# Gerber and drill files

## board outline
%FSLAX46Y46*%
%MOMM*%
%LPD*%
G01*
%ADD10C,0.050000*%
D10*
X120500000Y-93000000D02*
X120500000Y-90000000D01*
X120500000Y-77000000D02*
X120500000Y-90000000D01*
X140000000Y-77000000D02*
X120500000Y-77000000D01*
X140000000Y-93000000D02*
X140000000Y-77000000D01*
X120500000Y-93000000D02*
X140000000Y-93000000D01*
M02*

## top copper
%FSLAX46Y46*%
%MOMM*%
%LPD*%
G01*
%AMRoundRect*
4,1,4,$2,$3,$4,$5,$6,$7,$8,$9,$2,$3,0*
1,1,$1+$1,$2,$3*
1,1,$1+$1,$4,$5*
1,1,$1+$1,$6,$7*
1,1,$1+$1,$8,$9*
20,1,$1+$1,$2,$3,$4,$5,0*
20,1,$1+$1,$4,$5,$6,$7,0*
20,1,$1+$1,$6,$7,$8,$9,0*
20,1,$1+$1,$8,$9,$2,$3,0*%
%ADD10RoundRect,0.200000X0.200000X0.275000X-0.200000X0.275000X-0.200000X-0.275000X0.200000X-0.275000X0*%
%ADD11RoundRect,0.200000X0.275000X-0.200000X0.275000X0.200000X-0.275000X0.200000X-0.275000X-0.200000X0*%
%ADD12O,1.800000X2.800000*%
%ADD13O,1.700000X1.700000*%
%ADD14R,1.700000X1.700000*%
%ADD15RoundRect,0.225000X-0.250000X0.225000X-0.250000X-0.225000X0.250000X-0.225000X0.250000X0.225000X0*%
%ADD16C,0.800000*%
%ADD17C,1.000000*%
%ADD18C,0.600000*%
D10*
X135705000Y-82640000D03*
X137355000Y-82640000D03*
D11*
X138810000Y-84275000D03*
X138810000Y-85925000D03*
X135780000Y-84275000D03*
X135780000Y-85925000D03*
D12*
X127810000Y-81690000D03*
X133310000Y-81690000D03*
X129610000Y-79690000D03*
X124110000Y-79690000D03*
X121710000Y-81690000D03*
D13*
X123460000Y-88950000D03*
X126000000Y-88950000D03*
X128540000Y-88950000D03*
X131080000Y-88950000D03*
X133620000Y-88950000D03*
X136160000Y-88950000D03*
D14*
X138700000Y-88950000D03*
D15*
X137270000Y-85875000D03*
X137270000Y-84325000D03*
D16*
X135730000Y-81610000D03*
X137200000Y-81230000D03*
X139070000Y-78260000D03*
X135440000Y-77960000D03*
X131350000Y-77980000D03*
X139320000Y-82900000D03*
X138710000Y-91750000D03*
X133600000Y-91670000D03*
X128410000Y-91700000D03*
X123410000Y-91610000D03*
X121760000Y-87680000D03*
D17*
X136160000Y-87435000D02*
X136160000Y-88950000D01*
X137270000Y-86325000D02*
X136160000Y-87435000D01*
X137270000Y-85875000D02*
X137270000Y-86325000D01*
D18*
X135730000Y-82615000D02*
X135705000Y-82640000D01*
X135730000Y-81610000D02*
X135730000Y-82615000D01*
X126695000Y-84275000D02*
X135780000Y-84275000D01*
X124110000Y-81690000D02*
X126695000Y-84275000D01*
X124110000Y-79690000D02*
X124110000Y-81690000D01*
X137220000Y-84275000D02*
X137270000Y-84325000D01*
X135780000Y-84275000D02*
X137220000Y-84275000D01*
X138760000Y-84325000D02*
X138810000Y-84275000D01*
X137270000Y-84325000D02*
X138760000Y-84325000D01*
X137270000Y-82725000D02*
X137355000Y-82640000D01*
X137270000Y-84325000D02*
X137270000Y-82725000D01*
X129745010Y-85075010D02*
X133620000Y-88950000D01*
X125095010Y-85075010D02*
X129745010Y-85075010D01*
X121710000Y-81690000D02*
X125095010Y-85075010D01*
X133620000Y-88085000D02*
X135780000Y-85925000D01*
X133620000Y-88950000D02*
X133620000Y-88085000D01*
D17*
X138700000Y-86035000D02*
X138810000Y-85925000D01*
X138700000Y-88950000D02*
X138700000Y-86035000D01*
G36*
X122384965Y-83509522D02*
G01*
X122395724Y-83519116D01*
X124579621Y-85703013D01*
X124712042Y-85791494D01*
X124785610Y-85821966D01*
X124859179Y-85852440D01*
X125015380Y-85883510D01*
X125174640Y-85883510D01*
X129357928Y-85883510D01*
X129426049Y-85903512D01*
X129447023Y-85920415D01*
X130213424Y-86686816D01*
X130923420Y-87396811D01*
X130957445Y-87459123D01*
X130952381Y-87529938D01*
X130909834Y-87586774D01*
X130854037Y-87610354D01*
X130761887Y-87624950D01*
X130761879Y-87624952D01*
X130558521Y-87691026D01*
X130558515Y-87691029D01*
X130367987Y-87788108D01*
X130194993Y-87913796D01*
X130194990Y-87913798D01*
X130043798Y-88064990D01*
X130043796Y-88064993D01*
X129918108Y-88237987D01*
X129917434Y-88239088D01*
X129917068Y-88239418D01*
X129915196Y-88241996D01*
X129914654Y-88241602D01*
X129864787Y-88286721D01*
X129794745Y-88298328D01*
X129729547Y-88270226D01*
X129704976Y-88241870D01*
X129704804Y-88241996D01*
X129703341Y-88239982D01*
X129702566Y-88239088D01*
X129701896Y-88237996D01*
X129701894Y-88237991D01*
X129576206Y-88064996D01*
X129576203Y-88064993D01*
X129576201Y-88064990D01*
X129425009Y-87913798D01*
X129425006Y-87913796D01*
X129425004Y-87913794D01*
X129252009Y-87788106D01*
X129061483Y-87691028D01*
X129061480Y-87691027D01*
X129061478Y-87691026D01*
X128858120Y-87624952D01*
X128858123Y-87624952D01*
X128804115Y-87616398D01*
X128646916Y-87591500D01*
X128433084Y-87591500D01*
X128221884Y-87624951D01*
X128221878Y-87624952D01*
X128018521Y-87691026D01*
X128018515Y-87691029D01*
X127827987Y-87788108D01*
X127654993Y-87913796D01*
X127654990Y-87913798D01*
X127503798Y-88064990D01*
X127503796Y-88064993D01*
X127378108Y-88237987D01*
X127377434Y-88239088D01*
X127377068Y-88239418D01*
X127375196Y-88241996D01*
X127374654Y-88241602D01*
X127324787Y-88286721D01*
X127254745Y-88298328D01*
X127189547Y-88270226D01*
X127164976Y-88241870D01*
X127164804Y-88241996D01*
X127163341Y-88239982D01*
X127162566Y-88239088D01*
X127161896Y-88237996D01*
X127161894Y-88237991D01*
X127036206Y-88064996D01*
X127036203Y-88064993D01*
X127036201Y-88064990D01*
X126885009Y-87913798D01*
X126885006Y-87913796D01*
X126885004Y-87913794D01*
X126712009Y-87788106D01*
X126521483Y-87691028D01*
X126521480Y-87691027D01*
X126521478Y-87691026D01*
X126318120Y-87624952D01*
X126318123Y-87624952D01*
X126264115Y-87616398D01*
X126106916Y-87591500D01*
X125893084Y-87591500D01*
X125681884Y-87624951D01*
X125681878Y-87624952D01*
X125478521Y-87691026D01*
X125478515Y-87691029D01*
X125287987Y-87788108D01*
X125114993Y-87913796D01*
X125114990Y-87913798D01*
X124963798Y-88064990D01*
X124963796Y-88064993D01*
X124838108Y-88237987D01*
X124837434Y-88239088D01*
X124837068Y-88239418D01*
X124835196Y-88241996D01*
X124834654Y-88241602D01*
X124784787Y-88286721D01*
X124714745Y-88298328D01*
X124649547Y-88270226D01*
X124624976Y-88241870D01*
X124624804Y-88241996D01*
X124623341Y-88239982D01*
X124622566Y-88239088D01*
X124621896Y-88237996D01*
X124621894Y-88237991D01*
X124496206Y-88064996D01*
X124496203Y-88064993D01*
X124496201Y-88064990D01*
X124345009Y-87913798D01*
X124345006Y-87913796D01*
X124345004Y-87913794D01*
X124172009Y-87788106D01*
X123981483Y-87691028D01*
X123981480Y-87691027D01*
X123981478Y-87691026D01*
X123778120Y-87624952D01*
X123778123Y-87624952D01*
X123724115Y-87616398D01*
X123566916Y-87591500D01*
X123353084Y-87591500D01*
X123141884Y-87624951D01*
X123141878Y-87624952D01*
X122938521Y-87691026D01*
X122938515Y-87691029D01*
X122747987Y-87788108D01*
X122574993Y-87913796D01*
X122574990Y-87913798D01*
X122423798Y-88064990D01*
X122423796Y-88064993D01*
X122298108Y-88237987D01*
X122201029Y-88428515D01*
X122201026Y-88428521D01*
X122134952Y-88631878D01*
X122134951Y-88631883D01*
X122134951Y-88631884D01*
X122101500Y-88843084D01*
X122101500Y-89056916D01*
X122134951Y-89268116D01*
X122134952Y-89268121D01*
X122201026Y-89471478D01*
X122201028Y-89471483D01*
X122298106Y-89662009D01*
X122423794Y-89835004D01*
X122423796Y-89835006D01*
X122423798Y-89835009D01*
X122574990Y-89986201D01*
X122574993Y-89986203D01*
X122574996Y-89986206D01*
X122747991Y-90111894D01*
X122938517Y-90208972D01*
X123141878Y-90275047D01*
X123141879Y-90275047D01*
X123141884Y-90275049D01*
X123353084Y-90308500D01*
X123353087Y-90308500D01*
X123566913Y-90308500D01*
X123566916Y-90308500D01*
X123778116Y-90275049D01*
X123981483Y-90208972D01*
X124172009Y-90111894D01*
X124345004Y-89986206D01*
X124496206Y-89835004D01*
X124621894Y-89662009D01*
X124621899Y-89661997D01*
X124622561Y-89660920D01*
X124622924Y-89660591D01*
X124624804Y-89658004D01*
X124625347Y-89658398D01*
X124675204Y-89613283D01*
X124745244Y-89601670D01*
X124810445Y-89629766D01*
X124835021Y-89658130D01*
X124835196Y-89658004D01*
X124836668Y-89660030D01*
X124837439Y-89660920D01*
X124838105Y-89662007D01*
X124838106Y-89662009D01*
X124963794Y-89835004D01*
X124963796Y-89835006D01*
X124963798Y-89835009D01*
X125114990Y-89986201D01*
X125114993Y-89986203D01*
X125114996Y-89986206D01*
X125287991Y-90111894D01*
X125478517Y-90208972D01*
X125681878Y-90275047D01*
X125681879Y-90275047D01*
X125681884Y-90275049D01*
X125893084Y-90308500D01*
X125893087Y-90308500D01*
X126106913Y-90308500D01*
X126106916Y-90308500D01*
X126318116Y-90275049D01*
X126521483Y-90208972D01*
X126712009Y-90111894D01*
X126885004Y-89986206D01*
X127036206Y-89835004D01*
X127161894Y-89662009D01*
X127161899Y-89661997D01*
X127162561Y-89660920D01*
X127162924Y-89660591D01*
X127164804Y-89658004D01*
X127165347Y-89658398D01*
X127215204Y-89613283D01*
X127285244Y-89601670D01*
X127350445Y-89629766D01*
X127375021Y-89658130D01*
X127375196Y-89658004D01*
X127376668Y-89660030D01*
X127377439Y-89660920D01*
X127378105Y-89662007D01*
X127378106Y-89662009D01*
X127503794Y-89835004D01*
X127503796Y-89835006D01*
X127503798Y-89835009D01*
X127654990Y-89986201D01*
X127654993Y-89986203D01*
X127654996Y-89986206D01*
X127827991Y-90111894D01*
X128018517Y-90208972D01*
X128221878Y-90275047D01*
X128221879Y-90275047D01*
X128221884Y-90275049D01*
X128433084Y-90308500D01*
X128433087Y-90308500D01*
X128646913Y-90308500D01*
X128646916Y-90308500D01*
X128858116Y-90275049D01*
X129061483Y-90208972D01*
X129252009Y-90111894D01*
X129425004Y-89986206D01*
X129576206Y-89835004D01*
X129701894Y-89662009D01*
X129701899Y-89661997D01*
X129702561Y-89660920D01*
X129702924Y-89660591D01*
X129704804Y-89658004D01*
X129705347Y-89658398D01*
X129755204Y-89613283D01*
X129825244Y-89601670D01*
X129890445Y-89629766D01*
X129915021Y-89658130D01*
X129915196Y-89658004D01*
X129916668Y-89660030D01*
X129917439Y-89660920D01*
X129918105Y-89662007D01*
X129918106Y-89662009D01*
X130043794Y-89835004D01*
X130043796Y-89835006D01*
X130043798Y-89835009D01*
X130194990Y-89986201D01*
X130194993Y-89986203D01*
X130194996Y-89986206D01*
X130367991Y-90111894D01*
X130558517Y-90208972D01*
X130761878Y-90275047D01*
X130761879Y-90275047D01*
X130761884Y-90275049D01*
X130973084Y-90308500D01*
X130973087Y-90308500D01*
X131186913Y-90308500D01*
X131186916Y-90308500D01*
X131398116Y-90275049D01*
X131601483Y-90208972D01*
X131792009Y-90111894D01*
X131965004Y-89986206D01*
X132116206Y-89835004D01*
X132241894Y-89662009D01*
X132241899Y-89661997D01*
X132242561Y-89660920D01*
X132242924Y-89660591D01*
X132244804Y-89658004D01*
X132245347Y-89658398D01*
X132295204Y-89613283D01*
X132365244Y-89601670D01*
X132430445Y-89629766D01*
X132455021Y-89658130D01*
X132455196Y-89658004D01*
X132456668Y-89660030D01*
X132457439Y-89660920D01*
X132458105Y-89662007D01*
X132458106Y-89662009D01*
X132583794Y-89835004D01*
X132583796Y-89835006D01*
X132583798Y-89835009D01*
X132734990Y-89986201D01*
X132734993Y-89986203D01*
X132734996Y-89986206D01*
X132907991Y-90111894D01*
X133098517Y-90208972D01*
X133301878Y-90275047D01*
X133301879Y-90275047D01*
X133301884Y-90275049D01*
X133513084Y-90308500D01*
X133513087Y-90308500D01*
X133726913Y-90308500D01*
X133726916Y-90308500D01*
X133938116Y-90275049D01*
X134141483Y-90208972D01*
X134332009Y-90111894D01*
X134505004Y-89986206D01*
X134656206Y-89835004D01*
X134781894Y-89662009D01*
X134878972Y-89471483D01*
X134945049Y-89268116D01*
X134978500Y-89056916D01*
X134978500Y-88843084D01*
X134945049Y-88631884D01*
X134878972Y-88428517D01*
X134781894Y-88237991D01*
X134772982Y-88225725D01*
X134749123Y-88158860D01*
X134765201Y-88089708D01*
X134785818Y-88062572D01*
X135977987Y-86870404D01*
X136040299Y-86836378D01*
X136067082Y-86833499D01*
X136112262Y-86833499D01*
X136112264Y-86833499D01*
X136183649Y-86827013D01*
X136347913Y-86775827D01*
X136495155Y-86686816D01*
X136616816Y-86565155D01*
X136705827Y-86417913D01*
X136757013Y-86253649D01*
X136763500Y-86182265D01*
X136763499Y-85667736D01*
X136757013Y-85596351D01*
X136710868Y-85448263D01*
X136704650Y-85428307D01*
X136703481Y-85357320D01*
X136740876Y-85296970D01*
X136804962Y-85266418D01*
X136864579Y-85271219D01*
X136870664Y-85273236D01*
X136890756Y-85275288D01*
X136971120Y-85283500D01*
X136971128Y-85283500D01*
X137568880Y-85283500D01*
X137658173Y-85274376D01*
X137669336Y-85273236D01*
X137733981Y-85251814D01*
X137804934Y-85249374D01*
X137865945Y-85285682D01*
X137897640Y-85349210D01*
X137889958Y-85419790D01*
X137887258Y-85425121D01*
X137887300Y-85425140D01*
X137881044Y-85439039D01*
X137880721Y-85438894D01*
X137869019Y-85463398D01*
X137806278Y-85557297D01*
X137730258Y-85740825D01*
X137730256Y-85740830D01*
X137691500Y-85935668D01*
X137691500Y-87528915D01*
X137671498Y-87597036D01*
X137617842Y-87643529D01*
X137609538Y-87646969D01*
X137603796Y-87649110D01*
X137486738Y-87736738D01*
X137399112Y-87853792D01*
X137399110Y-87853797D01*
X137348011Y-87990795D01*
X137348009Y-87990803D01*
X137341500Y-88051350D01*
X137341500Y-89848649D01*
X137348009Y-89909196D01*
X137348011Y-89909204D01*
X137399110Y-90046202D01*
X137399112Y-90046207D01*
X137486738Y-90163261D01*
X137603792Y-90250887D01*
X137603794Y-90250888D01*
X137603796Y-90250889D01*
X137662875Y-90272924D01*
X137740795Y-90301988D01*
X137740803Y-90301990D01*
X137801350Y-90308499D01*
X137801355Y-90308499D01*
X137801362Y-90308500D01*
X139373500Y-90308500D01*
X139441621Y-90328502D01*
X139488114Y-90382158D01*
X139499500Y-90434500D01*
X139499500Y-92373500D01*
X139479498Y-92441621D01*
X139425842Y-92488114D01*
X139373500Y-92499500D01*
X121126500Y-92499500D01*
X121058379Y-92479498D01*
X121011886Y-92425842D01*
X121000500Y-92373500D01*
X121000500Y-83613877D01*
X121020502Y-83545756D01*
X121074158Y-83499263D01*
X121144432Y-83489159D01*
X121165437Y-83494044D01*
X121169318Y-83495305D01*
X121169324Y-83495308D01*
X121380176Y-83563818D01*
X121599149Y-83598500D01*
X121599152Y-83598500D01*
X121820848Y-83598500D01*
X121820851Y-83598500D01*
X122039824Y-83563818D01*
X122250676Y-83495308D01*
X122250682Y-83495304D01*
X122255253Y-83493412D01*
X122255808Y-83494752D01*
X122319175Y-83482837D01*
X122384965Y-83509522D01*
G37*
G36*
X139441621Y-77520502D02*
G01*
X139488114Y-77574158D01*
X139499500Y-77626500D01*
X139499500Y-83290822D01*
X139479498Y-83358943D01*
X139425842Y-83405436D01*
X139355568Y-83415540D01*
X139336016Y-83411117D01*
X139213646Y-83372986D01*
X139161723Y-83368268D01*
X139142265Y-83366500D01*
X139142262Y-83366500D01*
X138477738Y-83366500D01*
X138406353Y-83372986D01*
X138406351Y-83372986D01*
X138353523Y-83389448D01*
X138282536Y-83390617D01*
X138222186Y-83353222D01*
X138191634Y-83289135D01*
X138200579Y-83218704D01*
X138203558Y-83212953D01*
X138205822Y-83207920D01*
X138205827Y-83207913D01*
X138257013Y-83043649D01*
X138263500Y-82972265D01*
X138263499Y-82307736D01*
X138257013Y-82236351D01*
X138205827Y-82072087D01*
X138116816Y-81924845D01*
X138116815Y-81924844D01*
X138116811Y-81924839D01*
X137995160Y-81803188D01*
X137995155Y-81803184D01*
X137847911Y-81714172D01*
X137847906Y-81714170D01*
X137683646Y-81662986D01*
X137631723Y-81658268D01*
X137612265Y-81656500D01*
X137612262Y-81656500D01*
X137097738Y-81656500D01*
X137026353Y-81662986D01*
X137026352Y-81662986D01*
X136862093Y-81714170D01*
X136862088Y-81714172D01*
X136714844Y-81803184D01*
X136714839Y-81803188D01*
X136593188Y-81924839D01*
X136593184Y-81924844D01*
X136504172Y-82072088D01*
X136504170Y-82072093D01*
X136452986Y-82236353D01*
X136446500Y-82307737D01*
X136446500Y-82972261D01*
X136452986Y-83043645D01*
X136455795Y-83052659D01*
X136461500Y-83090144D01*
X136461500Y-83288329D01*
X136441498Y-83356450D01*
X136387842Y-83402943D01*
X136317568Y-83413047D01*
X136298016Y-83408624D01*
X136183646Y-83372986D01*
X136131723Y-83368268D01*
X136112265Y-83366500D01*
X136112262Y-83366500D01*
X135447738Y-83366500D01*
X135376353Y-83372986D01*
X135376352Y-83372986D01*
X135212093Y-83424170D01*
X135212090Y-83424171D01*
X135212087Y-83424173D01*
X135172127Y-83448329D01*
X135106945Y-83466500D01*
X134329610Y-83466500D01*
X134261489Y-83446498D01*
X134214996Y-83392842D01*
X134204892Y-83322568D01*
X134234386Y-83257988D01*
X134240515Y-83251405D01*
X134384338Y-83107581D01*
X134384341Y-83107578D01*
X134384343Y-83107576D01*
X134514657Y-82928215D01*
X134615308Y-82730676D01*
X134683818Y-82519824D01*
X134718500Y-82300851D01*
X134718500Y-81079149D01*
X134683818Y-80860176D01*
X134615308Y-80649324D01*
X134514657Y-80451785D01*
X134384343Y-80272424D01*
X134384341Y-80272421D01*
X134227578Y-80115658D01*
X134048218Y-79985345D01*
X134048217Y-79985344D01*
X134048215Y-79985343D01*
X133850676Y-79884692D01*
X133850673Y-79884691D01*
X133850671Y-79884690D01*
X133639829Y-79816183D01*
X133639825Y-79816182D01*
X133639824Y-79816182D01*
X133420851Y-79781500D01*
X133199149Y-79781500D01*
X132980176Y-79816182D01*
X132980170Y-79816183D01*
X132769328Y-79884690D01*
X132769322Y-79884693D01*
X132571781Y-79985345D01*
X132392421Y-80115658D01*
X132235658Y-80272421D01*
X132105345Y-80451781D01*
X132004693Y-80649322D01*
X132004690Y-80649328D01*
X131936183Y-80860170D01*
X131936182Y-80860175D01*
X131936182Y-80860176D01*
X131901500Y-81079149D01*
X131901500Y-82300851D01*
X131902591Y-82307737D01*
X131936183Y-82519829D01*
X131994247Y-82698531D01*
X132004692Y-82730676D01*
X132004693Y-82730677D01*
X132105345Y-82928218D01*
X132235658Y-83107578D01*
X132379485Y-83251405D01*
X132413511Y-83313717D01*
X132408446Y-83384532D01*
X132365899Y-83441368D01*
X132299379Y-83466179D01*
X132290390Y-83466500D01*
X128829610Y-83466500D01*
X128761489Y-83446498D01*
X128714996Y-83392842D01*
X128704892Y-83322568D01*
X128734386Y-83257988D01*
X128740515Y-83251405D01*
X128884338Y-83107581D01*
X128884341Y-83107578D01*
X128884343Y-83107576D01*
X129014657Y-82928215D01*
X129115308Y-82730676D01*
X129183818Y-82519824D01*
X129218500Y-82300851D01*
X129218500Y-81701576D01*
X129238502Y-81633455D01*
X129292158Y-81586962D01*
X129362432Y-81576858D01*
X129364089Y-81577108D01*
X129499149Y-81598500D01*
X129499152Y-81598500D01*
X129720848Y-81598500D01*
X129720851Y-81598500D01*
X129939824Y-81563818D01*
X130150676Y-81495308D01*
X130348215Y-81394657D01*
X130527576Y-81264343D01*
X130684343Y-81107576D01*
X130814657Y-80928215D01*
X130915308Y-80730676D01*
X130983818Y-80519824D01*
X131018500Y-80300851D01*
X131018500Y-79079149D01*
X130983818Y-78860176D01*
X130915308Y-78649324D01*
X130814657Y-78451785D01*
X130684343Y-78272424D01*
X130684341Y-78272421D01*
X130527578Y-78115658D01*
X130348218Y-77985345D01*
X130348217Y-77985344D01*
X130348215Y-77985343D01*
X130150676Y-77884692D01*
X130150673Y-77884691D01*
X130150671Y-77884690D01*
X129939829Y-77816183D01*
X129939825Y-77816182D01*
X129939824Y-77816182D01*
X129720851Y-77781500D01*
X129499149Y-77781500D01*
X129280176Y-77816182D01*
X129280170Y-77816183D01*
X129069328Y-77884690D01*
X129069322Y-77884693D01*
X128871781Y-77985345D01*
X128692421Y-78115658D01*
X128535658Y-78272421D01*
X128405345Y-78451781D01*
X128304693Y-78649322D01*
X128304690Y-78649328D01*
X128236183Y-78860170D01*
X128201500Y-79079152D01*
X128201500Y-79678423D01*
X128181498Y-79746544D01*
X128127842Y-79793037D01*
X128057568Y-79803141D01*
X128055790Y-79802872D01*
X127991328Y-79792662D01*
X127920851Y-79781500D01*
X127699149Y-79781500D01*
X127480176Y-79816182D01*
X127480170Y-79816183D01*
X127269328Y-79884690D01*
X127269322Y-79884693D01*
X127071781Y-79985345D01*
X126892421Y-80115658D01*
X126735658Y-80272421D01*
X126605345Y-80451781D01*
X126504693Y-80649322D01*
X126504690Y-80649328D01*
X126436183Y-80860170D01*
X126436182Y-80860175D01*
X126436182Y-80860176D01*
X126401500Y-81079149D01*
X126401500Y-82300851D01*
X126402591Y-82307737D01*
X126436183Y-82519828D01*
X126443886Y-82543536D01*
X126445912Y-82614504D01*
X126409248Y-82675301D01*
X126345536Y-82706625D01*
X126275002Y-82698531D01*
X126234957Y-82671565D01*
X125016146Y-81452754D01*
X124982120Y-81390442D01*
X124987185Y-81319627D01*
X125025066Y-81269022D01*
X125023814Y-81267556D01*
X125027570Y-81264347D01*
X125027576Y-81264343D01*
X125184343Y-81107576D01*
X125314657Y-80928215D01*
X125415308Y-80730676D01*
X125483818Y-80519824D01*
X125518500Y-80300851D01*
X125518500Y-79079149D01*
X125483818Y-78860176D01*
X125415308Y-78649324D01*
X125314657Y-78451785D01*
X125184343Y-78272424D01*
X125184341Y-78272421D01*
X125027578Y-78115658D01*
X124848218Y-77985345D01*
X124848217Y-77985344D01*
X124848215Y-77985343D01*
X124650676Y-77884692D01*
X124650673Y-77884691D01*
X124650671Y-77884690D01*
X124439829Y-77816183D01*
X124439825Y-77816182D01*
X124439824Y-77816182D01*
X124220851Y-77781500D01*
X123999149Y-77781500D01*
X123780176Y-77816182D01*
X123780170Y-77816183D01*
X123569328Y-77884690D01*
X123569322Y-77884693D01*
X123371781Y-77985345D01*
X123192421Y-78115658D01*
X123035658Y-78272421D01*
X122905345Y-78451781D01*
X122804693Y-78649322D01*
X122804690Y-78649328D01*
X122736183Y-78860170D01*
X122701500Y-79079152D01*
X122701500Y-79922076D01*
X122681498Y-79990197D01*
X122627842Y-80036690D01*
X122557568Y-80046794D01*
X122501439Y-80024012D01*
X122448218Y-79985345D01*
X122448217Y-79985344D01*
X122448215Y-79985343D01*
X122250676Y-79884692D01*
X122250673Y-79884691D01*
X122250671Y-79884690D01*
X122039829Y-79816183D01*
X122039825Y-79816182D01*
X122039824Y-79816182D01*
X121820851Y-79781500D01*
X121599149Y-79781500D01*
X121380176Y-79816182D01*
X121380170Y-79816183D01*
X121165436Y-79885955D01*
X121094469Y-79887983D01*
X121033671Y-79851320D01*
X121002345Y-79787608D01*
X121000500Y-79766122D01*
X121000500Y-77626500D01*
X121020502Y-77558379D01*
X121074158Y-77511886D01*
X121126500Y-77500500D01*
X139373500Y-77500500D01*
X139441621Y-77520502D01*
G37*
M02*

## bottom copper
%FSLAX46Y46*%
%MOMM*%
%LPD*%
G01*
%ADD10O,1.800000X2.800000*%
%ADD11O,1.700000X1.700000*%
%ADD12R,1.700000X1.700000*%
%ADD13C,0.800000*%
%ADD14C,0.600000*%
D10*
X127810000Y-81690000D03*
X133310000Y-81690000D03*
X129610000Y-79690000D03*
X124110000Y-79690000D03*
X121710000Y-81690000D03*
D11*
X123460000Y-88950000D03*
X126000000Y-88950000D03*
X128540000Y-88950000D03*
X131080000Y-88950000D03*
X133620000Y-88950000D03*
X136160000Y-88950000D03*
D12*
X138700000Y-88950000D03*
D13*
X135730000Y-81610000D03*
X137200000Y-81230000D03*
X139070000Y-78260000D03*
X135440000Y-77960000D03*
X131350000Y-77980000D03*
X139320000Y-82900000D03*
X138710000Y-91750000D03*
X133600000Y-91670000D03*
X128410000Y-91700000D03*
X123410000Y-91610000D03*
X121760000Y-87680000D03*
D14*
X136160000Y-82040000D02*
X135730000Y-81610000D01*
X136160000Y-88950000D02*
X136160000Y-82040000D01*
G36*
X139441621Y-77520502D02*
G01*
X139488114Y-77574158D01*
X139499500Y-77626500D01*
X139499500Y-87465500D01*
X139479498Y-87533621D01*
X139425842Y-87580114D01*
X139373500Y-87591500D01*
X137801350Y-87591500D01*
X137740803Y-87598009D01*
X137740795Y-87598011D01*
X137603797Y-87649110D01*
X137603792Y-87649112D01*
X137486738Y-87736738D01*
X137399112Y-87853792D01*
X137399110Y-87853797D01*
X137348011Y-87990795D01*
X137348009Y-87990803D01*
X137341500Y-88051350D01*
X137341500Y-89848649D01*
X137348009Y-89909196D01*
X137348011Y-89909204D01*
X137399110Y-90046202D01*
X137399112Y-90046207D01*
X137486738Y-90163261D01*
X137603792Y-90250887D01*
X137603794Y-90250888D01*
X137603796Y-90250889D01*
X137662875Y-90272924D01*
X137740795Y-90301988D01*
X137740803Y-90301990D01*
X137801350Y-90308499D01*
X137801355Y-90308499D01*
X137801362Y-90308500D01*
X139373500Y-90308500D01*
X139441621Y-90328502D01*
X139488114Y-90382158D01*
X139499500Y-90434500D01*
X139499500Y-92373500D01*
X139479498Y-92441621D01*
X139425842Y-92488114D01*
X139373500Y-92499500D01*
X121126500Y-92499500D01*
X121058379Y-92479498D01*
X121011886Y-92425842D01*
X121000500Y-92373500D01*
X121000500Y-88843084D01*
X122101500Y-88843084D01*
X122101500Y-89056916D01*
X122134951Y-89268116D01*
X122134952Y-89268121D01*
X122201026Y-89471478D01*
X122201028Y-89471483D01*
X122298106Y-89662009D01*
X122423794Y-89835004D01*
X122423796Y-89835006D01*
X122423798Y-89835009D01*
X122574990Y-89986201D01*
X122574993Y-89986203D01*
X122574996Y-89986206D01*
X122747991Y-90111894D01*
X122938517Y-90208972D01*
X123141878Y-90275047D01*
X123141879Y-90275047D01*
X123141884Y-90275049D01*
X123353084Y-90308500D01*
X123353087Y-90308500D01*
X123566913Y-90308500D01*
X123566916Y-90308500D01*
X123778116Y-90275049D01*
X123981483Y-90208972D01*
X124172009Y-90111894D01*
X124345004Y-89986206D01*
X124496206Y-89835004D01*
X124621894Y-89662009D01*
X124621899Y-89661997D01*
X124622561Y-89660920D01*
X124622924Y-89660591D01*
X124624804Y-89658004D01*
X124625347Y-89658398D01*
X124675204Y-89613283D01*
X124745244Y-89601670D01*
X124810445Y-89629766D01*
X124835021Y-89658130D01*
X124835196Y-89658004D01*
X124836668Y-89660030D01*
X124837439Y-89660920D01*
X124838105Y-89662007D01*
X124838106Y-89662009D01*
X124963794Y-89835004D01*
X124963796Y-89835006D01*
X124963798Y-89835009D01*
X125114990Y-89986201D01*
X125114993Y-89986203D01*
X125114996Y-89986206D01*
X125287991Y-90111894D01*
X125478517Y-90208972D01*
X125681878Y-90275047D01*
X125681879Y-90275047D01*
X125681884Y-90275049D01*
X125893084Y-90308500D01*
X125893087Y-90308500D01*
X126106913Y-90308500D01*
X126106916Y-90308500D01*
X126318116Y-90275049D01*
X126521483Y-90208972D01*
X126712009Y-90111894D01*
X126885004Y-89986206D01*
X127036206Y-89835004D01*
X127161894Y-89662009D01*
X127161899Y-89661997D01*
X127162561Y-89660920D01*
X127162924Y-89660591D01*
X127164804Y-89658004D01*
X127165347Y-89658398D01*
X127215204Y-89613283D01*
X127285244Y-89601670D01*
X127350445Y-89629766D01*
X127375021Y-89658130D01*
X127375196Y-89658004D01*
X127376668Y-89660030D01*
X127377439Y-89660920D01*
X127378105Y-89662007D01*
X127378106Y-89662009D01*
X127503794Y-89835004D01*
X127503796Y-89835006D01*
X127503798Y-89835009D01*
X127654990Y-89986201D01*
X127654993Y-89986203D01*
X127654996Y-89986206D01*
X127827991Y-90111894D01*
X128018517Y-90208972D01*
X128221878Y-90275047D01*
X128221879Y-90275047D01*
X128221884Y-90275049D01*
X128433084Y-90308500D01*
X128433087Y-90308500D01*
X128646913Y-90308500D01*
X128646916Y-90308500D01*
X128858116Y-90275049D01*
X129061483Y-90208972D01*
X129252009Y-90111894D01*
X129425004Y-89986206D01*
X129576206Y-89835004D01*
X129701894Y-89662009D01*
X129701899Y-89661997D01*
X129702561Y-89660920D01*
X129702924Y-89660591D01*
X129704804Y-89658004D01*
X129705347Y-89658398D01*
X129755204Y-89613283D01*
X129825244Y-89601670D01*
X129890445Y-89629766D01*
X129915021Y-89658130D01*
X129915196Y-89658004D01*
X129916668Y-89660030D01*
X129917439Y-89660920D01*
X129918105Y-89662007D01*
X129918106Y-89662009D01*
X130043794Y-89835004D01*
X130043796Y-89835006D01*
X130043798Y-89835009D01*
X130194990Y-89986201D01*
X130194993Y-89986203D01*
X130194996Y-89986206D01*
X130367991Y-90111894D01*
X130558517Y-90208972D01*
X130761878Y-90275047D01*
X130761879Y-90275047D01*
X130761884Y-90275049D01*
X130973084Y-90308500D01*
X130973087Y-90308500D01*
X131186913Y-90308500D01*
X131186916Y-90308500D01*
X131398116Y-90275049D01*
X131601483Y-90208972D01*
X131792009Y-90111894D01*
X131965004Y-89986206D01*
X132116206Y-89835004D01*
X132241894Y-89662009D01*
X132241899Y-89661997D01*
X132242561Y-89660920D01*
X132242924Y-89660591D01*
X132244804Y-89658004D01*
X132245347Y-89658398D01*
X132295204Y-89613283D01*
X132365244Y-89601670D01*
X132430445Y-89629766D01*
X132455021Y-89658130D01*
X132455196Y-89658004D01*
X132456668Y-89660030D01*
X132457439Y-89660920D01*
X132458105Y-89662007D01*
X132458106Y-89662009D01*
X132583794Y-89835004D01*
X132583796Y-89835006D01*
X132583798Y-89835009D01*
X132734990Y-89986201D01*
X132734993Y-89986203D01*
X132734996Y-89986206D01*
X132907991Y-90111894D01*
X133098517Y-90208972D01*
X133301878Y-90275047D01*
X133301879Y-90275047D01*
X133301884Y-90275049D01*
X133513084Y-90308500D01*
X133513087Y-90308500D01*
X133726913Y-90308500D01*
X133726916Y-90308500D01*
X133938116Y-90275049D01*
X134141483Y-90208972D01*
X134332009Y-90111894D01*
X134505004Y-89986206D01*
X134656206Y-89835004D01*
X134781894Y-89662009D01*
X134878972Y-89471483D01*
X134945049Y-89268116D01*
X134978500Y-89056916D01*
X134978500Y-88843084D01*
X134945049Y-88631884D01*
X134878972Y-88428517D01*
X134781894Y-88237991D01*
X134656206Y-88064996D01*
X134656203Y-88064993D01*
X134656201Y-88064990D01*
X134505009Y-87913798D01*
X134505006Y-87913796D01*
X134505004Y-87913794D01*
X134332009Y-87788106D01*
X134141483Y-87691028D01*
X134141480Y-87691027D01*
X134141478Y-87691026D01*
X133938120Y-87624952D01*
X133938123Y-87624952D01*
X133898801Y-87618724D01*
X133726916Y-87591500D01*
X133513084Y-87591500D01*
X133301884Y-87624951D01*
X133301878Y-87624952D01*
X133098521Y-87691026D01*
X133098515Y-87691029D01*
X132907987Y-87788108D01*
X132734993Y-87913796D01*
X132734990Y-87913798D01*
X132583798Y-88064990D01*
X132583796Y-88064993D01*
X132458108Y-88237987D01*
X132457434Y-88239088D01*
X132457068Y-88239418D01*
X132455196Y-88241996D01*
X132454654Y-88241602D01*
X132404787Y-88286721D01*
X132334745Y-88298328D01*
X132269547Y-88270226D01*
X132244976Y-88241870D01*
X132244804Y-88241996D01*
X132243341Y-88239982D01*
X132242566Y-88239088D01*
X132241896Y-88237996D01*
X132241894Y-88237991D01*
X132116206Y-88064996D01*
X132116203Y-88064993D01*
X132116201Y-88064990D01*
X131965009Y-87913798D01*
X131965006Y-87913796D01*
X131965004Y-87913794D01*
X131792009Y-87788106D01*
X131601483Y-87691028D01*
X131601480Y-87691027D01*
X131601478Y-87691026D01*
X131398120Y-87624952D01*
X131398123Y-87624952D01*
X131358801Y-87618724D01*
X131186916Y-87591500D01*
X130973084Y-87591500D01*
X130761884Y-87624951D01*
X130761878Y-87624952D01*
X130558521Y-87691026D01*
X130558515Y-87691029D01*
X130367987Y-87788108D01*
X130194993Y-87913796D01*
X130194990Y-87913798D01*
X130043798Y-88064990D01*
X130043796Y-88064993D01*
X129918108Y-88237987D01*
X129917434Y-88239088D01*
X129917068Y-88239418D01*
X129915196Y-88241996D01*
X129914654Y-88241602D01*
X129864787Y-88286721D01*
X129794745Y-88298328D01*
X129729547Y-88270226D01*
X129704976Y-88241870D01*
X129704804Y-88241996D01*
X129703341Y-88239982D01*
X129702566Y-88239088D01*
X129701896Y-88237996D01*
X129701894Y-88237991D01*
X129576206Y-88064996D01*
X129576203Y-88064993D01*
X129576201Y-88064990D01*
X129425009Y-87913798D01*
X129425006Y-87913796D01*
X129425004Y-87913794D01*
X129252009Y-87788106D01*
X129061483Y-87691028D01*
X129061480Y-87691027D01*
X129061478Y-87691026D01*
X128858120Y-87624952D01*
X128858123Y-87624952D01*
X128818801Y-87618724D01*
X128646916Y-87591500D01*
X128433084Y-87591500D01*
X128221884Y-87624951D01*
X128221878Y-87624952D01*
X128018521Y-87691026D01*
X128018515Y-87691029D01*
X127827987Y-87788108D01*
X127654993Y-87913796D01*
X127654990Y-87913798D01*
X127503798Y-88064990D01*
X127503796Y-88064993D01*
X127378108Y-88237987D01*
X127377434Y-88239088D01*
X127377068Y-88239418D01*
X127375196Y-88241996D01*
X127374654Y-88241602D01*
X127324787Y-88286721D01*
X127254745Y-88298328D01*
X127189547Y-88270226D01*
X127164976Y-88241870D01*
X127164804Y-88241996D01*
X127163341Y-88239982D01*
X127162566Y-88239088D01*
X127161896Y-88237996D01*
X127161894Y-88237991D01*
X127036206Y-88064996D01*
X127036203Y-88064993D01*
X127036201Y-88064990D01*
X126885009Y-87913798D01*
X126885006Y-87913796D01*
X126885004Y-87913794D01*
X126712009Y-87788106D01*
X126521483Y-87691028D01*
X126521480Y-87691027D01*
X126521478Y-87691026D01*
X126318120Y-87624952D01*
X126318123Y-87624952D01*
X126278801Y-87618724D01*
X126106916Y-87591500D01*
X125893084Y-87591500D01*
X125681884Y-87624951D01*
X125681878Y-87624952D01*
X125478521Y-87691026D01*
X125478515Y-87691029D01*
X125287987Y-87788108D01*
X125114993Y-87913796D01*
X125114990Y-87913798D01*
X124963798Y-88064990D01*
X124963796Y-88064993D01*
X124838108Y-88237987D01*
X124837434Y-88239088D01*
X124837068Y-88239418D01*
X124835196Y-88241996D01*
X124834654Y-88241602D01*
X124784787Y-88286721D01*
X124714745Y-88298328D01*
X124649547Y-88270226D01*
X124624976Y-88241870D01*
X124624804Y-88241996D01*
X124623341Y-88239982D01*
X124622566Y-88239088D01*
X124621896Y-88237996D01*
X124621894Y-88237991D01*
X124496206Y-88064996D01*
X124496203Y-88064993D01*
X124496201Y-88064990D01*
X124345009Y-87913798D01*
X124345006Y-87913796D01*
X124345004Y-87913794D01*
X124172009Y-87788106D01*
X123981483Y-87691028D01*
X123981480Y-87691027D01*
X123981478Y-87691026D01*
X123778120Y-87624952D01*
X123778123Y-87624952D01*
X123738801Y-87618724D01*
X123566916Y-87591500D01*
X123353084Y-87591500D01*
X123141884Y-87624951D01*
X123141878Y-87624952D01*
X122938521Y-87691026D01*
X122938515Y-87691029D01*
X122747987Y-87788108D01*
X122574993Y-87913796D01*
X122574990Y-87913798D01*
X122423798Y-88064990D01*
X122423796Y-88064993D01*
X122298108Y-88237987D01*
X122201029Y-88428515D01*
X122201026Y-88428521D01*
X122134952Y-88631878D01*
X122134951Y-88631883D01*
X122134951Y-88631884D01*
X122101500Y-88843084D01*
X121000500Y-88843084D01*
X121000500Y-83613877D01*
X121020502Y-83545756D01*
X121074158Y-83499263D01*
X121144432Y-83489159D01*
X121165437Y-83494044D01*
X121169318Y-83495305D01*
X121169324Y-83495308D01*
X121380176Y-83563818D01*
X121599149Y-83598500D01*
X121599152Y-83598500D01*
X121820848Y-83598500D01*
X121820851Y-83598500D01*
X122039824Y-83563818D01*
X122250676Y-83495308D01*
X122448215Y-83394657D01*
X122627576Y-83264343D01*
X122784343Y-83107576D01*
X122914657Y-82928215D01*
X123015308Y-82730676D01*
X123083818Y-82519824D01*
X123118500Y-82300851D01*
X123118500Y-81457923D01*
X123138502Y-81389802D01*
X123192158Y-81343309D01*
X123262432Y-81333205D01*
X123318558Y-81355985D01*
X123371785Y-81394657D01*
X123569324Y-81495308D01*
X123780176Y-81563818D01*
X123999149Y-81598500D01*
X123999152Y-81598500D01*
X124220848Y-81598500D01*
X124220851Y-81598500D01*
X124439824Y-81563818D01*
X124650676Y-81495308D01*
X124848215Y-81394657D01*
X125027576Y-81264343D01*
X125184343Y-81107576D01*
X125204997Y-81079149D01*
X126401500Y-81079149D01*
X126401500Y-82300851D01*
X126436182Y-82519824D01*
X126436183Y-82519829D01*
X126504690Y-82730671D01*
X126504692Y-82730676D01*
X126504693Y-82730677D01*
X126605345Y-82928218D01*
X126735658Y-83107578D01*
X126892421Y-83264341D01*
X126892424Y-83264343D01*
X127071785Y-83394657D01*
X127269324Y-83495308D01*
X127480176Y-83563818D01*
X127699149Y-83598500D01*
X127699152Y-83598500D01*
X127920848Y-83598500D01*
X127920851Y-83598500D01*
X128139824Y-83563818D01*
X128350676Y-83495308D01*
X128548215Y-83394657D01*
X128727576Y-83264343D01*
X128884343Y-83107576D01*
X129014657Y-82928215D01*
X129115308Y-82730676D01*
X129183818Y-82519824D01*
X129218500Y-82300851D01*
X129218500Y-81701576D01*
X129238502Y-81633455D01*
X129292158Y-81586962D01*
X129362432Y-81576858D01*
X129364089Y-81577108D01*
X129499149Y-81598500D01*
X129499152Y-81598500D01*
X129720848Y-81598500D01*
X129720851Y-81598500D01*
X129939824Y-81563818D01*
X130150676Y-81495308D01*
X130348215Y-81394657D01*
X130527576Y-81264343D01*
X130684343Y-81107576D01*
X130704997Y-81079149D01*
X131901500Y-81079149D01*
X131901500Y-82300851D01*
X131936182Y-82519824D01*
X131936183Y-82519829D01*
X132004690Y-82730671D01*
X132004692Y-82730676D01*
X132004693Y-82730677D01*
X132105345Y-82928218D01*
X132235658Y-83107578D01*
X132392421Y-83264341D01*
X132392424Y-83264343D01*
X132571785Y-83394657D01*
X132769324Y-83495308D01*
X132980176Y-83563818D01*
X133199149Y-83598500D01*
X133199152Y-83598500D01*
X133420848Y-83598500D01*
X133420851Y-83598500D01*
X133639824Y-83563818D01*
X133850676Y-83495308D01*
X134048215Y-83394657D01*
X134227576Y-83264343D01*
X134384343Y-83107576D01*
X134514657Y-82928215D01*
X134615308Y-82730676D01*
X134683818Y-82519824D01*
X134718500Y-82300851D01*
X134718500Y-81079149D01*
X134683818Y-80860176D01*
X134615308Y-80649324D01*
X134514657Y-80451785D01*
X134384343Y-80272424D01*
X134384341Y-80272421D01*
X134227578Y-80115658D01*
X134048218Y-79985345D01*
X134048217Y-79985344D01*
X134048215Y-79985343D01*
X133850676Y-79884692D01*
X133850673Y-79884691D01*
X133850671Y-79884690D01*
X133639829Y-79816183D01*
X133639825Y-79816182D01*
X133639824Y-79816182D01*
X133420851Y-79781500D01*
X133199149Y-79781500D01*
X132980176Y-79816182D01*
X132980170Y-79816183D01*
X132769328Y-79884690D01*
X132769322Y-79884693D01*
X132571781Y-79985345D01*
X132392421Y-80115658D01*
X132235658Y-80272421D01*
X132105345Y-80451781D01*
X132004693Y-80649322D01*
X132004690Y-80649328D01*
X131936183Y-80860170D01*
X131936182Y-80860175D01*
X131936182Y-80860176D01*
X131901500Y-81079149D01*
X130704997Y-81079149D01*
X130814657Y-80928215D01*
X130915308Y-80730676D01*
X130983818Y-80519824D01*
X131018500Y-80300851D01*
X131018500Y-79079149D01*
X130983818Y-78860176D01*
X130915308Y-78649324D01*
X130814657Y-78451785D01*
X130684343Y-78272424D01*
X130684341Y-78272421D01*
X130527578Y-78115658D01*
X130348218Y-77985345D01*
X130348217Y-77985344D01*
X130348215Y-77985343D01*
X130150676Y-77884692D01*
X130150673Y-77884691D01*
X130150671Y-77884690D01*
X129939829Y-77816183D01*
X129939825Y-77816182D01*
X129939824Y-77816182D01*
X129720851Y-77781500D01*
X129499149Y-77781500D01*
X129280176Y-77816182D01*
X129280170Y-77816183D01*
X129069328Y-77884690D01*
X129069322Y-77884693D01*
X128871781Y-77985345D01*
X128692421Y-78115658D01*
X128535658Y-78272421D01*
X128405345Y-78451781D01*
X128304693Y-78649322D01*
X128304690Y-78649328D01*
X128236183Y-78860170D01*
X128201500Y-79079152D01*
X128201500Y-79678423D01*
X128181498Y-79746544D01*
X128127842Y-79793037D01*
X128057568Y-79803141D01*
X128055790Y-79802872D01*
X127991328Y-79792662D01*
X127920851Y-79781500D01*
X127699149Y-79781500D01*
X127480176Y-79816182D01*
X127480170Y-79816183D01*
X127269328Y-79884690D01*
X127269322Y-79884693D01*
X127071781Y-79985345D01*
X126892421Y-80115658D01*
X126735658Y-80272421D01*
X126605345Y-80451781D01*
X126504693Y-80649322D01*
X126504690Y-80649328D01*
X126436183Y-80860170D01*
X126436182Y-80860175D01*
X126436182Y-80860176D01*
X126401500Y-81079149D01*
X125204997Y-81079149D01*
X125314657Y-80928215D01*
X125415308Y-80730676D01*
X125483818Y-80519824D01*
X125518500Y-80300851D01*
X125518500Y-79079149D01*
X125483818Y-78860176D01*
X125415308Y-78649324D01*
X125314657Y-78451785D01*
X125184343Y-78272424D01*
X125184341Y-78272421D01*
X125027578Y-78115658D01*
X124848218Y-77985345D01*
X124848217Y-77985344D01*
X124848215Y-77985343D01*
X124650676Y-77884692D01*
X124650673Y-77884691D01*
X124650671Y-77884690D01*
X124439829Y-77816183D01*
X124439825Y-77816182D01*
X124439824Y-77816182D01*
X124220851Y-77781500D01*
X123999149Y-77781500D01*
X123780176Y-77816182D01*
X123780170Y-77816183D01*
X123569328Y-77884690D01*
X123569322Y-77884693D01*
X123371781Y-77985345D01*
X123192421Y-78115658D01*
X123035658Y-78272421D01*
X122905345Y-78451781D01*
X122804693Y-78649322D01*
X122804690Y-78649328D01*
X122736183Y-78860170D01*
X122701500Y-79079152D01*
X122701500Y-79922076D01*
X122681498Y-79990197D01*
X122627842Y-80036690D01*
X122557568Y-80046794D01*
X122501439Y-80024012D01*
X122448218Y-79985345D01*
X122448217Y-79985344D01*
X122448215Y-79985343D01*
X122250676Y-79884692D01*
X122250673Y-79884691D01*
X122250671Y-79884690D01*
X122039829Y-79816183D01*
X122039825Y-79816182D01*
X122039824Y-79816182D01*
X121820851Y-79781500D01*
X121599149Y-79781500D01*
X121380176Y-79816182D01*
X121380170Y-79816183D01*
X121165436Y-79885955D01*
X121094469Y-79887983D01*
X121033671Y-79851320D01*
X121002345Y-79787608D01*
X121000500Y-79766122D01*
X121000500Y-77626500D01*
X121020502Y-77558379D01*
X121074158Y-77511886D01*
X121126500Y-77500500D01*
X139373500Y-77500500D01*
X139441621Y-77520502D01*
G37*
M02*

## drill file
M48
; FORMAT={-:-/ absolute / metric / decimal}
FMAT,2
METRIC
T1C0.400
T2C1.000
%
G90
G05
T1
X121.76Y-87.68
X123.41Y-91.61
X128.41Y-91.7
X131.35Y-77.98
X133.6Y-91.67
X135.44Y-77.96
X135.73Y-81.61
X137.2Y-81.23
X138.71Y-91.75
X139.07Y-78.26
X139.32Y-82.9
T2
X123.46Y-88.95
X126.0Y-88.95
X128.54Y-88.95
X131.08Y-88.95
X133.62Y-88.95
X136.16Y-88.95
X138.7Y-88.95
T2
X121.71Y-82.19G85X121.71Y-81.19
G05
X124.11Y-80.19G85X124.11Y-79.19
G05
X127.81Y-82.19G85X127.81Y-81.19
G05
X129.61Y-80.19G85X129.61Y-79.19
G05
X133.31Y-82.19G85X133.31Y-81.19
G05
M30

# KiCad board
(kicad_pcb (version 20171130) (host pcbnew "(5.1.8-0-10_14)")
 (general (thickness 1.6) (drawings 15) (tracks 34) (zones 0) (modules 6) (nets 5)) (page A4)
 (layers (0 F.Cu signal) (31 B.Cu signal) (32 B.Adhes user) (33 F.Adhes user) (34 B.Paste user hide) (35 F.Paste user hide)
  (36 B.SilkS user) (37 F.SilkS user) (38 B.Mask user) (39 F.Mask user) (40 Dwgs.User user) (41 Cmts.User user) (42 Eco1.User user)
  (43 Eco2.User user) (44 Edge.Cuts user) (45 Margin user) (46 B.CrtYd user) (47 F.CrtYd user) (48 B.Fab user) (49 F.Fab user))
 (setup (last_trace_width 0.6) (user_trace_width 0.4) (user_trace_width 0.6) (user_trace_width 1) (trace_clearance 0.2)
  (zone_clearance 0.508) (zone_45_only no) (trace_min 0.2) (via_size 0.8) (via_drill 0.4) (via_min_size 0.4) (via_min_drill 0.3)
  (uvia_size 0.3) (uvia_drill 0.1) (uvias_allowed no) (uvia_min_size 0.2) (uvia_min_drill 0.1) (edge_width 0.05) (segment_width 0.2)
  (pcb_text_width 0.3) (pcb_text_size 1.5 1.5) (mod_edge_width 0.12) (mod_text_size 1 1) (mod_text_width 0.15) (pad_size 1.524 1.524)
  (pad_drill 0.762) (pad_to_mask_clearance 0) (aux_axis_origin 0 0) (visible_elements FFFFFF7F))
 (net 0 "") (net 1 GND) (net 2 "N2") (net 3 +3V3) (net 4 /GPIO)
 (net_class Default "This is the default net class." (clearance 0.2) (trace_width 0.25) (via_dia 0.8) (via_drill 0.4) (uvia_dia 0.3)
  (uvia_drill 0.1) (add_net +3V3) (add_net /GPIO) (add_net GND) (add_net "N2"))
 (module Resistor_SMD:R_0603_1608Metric (layer F.Cu) (at 136.53 82.64 180)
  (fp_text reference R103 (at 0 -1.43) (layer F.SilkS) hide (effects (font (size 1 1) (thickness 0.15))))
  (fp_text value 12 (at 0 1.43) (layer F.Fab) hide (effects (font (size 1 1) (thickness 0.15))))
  (pad 2 smd roundrect (at 0.825 0 180) (size 0.8 0.95) (layers F.Cu F.Paste F.Mask) (roundrect_rratio 0.25) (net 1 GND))
  (pad 1 smd roundrect (at -0.825 0 180) (size 0.8 0.95) (layers F.Cu F.Paste F.Mask) (roundrect_rratio 0.25) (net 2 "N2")))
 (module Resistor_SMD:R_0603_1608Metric (layer F.Cu) (at 138.81 85.1 90)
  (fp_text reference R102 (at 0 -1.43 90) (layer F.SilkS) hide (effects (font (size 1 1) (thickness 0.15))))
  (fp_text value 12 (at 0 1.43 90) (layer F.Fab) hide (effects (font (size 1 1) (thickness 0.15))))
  (pad 2 smd roundrect (at 0.825 0 90) (size 0.8 0.95) (layers F.Cu F.Paste F.Mask) (roundrect_rratio 0.25) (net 2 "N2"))
  (pad 1 smd roundrect (at -0.825 0 90) (size 0.8 0.95) (layers F.Cu F.Paste F.Mask) (roundrect_rratio 0.25) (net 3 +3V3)))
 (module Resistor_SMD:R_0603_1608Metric (layer F.Cu) (at 135.78 85.1 90)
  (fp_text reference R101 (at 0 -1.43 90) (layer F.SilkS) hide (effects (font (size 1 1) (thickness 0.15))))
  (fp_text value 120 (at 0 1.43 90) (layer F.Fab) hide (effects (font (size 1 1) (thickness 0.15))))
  (pad 2 smd roundrect (at 0.825 0 90) (size 0.8 0.95) (layers F.Cu F.Paste F.Mask) (roundrect_rratio 0.25) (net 2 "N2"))
  (pad 1 smd roundrect (at -0.825 0 90) (size 0.8 0.95) (layers F.Cu F.Paste F.Mask) (roundrect_rratio 0.25) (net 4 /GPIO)))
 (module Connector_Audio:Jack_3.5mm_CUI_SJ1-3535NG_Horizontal (layer F.Cu) (at 121.71 81.69 90)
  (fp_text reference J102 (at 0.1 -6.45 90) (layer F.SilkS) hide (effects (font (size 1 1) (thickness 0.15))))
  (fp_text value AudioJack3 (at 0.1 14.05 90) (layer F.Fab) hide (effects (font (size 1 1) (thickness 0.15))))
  (pad RN thru_hole oval (at 0 6.1 90) (size 2.8 1.8) (drill oval 2 1) (layers *.Cu *.Mask))
  (pad TN thru_hole oval (at 0 11.6 90) (size 2.8 1.8) (drill oval 2 1) (layers *.Cu *.Mask))
  (pad R thru_hole oval (at 2 7.9 90) (size 2.8 1.8) (drill oval 2 1) (layers *.Cu *.Mask))
  (pad T thru_hole oval (at 2 2.4 90) (size 2.8 1.8) (drill oval 2 1) (layers *.Cu *.Mask) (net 2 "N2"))
  (pad S thru_hole oval (at 0 0 90) (size 2.8 1.8) (drill oval 2 1) (layers *.Cu *.Mask) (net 4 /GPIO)))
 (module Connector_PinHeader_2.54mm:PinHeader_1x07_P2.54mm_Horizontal (layer F.Cu) (at 138.7 88.95 270)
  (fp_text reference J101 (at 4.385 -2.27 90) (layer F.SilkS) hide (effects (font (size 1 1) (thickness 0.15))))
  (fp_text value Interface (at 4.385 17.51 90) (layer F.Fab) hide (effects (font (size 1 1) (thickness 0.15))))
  (pad 7 thru_hole oval (at 0 15.24 270) (size 1.7 1.7) (drill 1) (layers *.Cu *.Mask))
  (pad 6 thru_hole oval (at 0 12.7 270) (size 1.7 1.7) (drill 1) (layers *.Cu *.Mask))
  (pad 5 thru_hole oval (at 0 10.16 270) (size 1.7 1.7) (drill 1) (layers *.Cu *.Mask))
  (pad 4 thru_hole oval (at 0 7.62 270) (size 1.7 1.7) (drill 1) (layers *.Cu *.Mask))
  (pad 3 thru_hole oval (at 0 5.08 270) (size 1.7 1.7) (drill 1) (layers *.Cu *.Mask) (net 4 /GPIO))
  (pad 2 thru_hole oval (at 0 2.54 270) (size 1.7 1.7) (drill 1) (layers *.Cu *.Mask) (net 1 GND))
  (pad 1 thru_hole rect (at 0 0 270) (size 1.7 1.7) (drill 1) (layers *.Cu *.Mask) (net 3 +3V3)))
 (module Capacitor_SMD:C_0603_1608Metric (layer F.Cu) (at 137.27 85.1 270)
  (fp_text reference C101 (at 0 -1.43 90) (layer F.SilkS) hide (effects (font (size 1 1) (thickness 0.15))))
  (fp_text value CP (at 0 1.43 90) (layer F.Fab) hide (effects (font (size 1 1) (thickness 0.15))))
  (pad 2 smd roundrect (at 0.775 0 270) (size 0.9 0.95) (layers F.Cu F.Paste F.Mask) (roundrect_rratio 0.25) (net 1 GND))
  (pad 1 smd roundrect (at -0.775 0 270) (size 0.9 0.95) (layers F.Cu F.Paste F.Mask) (roundrect_rratio 0.25) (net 2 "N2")))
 (gr_line (start 120.5 93) (end 120.5 90) (layer Edge.Cuts) (width 0.05))
 (gr_line (start 120.5 77) (end 120.5 90) (layer Edge.Cuts) (width 0.05))
 (gr_line (start 140 77) (end 120.5 77) (layer Edge.Cuts) (width 0.05))
 (gr_line (start 140 93) (end 140 77) (layer Edge.Cuts) (width 0.05))
 (gr_line (start 120.5 93) (end 140 93) (layer Edge.Cuts) (width 0.05))
 (segment (start 136.16 87.435) (end 136.16 88.95) (width 1) (layer F.Cu) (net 1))
 (segment (start 137.27 86.325) (end 136.16 87.435) (width 1) (layer F.Cu) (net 1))
 (segment (start 137.27 85.875) (end 137.27 86.325) (width 1) (layer F.Cu) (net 1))
 (segment (start 136.16 82.04) (end 135.73 81.61) (width 0.6) (layer B.Cu) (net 1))
 (via (at 135.73 81.61) (size 0.8) (drill 0.4) (layers F.Cu B.Cu) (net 1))
 (segment (start 136.16 88.95) (end 136.16 82.04) (width 0.6) (layer B.Cu) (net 1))
 (segment (start 135.73 82.615) (end 135.705 82.64) (width 0.6) (layer F.Cu) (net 1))
 (segment (start 135.73 81.61) (end 135.73 82.615) (width 0.6) (layer F.Cu) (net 1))
 (via (at 137.2 81.23) (size 0.8) (drill 0.4) (layers F.Cu B.Cu) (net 1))
 (via (at 139.07 78.26) (size 0.8) (drill 0.4) (layers F.Cu B.Cu) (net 1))
 (via (at 135.44 77.96) (size 0.8) (drill 0.4) (layers F.Cu B.Cu) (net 1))
 (via (at 131.35 77.98) (size 0.8) (drill 0.4) (layers F.Cu B.Cu) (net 1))
 (via (at 139.32 82.9) (size 0.8) (drill 0.4) (layers F.Cu B.Cu) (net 1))
 (via (at 138.71 91.75) (size 0.8) (drill 0.4) (layers F.Cu B.Cu) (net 1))
 (via (at 133.6 91.67) (size 0.8) (drill 0.4) (layers F.Cu B.Cu) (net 1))
 (via (at 128.41 91.7) (size 0.8) (drill 0.4) (layers F.Cu B.Cu) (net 1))
 (via (at 123.41 91.61) (size 0.8) (drill 0.4) (layers F.Cu B.Cu) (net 1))
 (via (at 121.76 87.68) (size 0.8) (drill 0.4) (layers F.Cu B.Cu) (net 1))
 (segment (start 126.695 84.275) (end 135.78 84.275) (width 0.6) (layer F.Cu) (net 2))
 (segment (start 124.11 81.69) (end 126.695 84.275) (width 0.6) (layer F.Cu) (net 2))
 (segment (start 124.11 79.69) (end 124.11 81.69) (width 0.6) (layer F.Cu) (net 2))
 (segment (start 137.22 84.275) (end 137.27 84.325) (width 0.6) (layer F.Cu) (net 2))
 (segment (start 135.78 84.275) (end 137.22 84.275) (width 0.6) (layer F.Cu) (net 2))
 (segment (start 138.76 84.325) (end 138.81 84.275) (width 0.6) (layer F.Cu) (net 2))
 (segment (start 137.27 84.325) (end 138.76 84.325) (width 0.6) (layer F.Cu) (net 2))
 (segment (start 137.27 82.725) (end 137.355 82.64) (width 0.6) (layer F.Cu) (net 2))
 (segment (start 137.27 84.325) (end 137.27 82.725) (width 0.6) (layer F.Cu) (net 2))
 (segment (start 129.74501 85.07501) (end 133.62 88.95) (width 0.6) (layer F.Cu) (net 4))
 (segment (start 125.09501 85.07501) (end 129.74501 85.07501) (width 0.6) (layer F.Cu) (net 4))
 (segment (start 121.71 81.69) (end 125.09501 85.07501) (width 0.6) (layer F.Cu) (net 4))
 (segment (start 133.62 88.085) (end 135.78 85.925) (width 0.6) (layer F.Cu) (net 4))
 (segment (start 133.62 88.95) (end 133.62 88.085) (width 0.6) (layer F.Cu) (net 4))
 (segment (start 138.7 86.035) (end 138.81 85.925) (width 1) (layer F.Cu) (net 3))
 (segment (start 138.7 88.95) (end 138.7 86.035) (width 1) (layer F.Cu) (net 3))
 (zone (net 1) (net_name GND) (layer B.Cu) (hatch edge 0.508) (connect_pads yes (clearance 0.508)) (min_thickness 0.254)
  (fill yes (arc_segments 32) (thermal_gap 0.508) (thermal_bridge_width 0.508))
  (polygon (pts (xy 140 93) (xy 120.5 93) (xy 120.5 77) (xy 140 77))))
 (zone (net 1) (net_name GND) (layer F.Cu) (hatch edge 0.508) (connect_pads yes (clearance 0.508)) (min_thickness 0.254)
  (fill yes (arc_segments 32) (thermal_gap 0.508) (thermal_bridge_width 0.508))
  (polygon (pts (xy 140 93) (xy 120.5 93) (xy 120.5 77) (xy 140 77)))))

